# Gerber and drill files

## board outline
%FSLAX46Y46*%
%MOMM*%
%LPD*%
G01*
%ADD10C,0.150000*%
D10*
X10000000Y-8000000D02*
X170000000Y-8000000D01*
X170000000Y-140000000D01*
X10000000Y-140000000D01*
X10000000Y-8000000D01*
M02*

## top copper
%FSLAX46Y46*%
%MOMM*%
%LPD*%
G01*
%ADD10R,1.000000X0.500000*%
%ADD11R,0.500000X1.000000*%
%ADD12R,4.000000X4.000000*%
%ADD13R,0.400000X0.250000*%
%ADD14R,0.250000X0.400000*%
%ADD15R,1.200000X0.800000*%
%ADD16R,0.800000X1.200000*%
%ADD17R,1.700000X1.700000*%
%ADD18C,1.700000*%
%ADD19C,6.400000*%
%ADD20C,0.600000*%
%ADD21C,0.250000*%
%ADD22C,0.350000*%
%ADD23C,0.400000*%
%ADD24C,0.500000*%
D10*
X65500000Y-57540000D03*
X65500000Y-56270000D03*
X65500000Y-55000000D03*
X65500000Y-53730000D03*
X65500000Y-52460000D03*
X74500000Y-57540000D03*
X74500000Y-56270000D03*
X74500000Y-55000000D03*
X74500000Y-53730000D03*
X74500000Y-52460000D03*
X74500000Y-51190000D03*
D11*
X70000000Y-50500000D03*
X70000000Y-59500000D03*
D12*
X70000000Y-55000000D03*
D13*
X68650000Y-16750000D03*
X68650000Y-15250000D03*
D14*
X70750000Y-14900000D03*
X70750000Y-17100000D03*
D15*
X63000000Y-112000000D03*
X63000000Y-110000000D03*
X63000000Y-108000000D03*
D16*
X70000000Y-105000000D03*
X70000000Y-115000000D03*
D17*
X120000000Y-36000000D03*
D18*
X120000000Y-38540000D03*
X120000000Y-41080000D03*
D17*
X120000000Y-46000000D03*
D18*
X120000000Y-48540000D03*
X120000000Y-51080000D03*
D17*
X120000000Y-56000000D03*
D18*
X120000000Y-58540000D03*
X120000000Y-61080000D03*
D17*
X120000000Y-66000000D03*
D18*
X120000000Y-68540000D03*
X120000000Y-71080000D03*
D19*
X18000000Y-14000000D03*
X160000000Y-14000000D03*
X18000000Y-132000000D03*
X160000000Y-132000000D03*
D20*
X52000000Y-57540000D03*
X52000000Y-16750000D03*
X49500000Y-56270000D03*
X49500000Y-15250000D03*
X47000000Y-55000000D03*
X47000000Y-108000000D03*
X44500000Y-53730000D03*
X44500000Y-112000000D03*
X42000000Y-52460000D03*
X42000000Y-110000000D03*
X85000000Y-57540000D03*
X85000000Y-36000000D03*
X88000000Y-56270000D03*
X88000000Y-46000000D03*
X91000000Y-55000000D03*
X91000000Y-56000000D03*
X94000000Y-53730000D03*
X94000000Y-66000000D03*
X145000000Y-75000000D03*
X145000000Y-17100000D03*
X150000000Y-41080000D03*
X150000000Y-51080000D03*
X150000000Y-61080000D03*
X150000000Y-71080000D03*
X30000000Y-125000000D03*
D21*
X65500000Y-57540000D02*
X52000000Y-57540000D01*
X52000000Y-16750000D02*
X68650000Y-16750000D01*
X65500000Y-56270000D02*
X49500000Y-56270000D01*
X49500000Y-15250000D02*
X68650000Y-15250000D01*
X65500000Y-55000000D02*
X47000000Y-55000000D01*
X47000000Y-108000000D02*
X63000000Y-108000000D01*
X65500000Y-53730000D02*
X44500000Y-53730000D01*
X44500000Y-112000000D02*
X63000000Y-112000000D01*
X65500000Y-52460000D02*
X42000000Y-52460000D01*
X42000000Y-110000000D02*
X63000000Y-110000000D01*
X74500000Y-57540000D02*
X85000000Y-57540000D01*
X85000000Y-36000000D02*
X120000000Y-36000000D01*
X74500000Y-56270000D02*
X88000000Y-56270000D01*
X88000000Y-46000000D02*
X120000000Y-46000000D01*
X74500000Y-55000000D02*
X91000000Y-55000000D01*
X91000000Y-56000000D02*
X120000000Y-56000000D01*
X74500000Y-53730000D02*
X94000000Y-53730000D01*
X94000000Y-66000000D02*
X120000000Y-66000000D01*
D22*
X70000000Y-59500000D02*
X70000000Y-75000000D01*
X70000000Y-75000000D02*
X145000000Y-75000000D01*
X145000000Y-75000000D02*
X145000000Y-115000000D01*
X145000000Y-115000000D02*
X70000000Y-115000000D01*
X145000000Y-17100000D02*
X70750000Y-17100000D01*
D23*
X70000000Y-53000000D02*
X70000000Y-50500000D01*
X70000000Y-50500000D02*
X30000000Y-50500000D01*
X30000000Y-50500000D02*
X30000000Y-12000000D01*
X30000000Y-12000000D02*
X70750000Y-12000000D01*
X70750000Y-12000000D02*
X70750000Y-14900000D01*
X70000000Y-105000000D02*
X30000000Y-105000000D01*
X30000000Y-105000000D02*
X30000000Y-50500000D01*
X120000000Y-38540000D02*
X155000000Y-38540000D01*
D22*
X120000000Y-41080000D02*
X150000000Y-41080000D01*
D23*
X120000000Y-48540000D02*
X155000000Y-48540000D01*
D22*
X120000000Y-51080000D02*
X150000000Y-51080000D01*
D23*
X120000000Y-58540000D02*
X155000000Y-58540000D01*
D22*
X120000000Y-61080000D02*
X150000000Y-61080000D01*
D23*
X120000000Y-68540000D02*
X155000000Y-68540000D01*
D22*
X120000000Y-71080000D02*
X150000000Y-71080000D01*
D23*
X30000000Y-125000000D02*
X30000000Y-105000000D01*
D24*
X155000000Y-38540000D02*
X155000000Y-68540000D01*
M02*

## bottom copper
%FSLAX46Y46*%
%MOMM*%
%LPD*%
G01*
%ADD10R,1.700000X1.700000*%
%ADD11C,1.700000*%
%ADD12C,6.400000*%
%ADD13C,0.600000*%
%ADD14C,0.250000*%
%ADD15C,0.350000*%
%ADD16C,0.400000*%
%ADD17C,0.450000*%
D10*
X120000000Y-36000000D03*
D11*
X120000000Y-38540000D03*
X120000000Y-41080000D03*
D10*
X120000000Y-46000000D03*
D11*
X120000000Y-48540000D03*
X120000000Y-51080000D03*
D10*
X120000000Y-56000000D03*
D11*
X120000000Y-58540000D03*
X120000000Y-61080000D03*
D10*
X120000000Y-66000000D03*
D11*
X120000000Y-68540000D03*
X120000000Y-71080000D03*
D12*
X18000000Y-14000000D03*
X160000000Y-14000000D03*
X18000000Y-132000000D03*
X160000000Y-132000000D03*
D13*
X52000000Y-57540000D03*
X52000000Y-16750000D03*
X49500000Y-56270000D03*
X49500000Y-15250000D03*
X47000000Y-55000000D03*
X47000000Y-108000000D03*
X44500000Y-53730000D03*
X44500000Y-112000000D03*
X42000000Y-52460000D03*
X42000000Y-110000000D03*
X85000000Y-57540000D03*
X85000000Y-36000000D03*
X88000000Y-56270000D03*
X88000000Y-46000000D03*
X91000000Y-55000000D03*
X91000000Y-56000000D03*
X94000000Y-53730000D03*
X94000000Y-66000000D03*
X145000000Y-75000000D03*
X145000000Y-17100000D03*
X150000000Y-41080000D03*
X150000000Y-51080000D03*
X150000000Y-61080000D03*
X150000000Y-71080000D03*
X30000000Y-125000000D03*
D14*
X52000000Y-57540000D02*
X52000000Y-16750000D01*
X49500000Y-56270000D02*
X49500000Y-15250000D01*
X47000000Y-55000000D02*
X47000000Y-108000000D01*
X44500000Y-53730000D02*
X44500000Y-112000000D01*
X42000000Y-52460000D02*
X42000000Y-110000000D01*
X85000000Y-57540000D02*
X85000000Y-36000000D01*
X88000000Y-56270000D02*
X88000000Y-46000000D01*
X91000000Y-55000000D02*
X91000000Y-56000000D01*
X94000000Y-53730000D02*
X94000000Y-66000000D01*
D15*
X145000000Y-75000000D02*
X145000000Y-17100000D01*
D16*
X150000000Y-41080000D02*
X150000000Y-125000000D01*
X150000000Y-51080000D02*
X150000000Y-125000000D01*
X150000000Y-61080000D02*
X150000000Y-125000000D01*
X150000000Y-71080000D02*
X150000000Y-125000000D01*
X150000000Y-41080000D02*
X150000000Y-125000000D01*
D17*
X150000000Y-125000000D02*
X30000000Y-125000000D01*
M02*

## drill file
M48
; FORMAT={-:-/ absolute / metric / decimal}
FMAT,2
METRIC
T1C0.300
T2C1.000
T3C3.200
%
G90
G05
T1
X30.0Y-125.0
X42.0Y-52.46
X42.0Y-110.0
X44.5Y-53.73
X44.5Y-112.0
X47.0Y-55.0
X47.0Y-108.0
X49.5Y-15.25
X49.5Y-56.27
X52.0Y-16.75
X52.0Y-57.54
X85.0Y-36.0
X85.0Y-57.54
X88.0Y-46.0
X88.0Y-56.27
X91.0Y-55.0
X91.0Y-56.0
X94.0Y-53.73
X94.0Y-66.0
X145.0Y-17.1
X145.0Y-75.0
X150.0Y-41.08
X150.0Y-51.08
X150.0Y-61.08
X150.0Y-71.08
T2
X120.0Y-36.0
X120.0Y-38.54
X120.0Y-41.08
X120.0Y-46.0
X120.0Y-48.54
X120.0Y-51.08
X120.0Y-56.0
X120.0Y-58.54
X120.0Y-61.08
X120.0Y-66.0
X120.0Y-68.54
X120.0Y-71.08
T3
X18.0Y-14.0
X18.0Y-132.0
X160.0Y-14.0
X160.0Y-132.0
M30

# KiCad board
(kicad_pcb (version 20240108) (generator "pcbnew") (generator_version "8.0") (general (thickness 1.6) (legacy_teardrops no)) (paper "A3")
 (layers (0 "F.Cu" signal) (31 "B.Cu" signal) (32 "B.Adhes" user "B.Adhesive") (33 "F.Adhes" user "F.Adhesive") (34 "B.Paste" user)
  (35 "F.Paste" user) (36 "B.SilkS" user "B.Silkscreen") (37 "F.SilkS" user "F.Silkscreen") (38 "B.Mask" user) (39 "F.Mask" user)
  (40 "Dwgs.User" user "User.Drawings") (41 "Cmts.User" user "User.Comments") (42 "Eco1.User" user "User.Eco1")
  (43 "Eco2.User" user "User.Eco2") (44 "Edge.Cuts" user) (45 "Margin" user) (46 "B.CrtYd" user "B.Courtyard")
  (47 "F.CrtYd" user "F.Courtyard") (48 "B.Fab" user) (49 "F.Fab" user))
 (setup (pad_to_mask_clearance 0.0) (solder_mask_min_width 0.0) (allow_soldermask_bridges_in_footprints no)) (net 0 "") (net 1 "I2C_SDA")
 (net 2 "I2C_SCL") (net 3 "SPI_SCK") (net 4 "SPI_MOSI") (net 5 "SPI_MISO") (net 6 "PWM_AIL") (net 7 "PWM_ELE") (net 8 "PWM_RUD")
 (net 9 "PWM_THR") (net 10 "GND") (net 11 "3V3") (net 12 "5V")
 (gr_rect (start 10 8) (end 170 140) (stroke (width 0.15) (type solid)) (fill none) (layer "Edge.Cuts"))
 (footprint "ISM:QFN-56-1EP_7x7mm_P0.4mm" (layer "F.Cu") (at 70 55)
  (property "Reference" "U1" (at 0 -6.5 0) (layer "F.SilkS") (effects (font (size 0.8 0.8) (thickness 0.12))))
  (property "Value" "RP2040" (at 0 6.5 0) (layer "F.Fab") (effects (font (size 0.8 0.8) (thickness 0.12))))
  (pad "1" smd rect (at -4.5 2.54) (size 1.0 0.5) (layers "F.Cu" "F.Paste" "F.Mask") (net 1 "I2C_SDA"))
  (pad "2" smd rect (at -4.5 1.27) (size 1.0 0.5) (layers "F.Cu" "F.Paste" "F.Mask") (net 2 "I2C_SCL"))
  (pad "3" smd rect (at -4.5 0) (size 1.0 0.5) (layers "F.Cu" "F.Paste" "F.Mask") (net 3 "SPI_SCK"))
  (pad "4" smd rect (at -4.5 -1.27) (size 1.0 0.5) (layers "F.Cu" "F.Paste" "F.Mask") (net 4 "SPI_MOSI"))
  (pad "5" smd rect (at -4.5 -2.54) (size 1.0 0.5) (layers "F.Cu" "F.Paste" "F.Mask") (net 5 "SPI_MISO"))
  (pad "6" smd rect (at 4.5 2.54) (size 1.0 0.5) (layers "F.Cu" "F.Paste" "F.Mask") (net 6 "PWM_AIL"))
  (pad "7" smd rect (at 4.5 1.27) (size 1.0 0.5) (layers "F.Cu" "F.Paste" "F.Mask") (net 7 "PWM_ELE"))
  (pad "8" smd rect (at 4.5 0) (size 1.0 0.5) (layers "F.Cu" "F.Paste" "F.Mask") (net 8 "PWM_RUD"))
  (pad "9" smd rect (at 4.5 -1.27) (size 1.0 0.5) (layers "F.Cu" "F.Paste" "F.Mask") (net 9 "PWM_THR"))
  (pad "12" smd rect (at 4.5 -2.54) (size 1.0 0.5) (layers "F.Cu" "F.Paste" "F.Mask"))
  (pad "13" smd rect (at 4.5 -3.81) (size 1.0 0.5) (layers "F.Cu" "F.Paste" "F.Mask"))
  (pad "10" smd rect (at 0 -4.5) (size 0.5 1.0) (layers "F.Cu" "F.Paste" "F.Mask") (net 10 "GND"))
  (pad "11" smd rect (at 0 4.5) (size 0.5 1.0) (layers "F.Cu" "F.Paste" "F.Mask") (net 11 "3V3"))
  (pad "EP" smd rect (at 0 0) (size 4 4) (layers "F.Cu" "F.Paste" "F.Mask") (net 10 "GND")))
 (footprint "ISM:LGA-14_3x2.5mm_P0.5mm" (layer "F.Cu") (at 70 16)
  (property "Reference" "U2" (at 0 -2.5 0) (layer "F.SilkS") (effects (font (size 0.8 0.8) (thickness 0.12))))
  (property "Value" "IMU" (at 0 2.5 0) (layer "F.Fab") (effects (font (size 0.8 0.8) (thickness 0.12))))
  (pad "1" smd rect (at -1.35 0.75) (size 0.4 0.25) (layers "F.Cu" "F.Paste" "F.Mask") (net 1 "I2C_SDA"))
  (pad "2" smd rect (at -1.35 -0.75) (size 0.4 0.25) (layers "F.Cu" "F.Paste" "F.Mask") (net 2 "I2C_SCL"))
  (pad "3" smd rect (at 0.75 -1.1) (size 0.25 0.4) (layers "F.Cu" "F.Paste" "F.Mask") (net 10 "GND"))
  (pad "4" smd rect (at 0.75 1.1) (size 0.25 0.4) (layers "F.Cu" "F.Paste" "F.Mask") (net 11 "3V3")))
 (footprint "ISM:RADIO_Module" (layer "F.Cu") (at 70 110)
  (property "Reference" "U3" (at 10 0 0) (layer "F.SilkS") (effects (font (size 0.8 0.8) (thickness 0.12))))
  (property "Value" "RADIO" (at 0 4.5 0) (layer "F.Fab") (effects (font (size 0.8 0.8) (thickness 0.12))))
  (pad "1" smd rect (at -7 2) (size 1.2 0.8) (layers "F.Cu" "F.Paste" "F.Mask") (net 4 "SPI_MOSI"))
  (pad "2" smd rect (at -7 0) (size 1.2 0.8) (layers "F.Cu" "F.Paste" "F.Mask") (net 5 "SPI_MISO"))
  (pad "3" smd rect (at -7 -2) (size 1.2 0.8) (layers "F.Cu" "F.Paste" "F.Mask") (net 3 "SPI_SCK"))
  (pad "4" smd rect (at 0 -5) (size 0.8 1.2) (layers "F.Cu" "F.Paste" "F.Mask") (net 10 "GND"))
  (pad "5" smd rect (at 0 5) (size 0.8 1.2) (layers "F.Cu" "F.Paste" "F.Mask") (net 11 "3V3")))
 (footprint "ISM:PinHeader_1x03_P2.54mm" (layer "F.Cu") (at 120 36)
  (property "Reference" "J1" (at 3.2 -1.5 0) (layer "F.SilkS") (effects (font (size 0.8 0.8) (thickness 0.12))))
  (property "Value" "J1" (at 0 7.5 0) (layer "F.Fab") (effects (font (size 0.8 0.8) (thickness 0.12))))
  (pad "1" thru_hole rect (at 0 0) (size 1.7 1.7) (drill 1.0) (layers "*.Cu" "*.Mask") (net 6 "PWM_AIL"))
  (pad "2" thru_hole circle (at 0 2.54) (size 1.7 1.7) (drill 1.0) (layers "*.Cu" "*.Mask") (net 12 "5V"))
  (pad "3" thru_hole circle (at 0 5.08) (size 1.7 1.7) (drill 1.0) (layers "*.Cu" "*.Mask") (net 10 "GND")))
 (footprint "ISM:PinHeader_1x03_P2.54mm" (layer "F.Cu") (at 120 46)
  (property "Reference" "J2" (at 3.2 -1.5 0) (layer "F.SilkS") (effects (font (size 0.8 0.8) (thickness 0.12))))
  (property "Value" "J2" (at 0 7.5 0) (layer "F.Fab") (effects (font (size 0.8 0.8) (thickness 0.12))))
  (pad "1" thru_hole rect (at 0 0) (size 1.7 1.7) (drill 1.0) (layers "*.Cu" "*.Mask") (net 7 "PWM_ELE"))
  (pad "2" thru_hole circle (at 0 2.54) (size 1.7 1.7) (drill 1.0) (layers "*.Cu" "*.Mask") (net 12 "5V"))
  (pad "3" thru_hole circle (at 0 5.08) (size 1.7 1.7) (drill 1.0) (layers "*.Cu" "*.Mask") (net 10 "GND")))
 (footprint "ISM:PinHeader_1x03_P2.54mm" (layer "F.Cu") (at 120 56)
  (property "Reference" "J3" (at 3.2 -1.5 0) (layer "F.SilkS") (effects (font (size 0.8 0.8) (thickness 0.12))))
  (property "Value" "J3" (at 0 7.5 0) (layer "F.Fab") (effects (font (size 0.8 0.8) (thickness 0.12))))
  (pad "1" thru_hole rect (at 0 0) (size 1.7 1.7) (drill 1.0) (layers "*.Cu" "*.Mask") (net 8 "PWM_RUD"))
  (pad "2" thru_hole circle (at 0 2.54) (size 1.7 1.7) (drill 1.0) (layers "*.Cu" "*.Mask") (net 12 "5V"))
  (pad "3" thru_hole circle (at 0 5.08) (size 1.7 1.7) (drill 1.0) (layers "*.Cu" "*.Mask") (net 10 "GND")))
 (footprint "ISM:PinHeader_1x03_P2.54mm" (layer "F.Cu") (at 120 66)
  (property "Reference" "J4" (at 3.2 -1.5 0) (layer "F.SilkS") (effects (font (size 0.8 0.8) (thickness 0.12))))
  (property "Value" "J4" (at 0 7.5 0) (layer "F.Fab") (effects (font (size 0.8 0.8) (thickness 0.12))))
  (pad "1" thru_hole rect (at 0 0) (size 1.7 1.7) (drill 1.0) (layers "*.Cu" "*.Mask") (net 9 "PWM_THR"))
  (pad "2" thru_hole circle (at 0 2.54) (size 1.7 1.7) (drill 1.0) (layers "*.Cu" "*.Mask") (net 12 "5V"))
  (pad "3" thru_hole circle (at 0 5.08) (size 1.7 1.7) (drill 1.0) (layers "*.Cu" "*.Mask") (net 10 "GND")))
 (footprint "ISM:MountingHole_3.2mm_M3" (layer "F.Cu") (at 18 14)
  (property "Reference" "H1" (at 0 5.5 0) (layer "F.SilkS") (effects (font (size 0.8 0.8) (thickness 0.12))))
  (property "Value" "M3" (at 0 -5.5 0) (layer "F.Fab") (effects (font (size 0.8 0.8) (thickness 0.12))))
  (pad "" thru_hole circle (at 0 0) (size 6.4 6.4) (drill 3.2) (layers "*.Cu" "*.Mask")))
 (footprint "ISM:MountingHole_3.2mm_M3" (layer "F.Cu") (at 160 14)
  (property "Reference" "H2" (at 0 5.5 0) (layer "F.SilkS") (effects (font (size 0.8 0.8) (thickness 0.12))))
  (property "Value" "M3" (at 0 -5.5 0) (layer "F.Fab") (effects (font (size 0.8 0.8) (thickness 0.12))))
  (pad "" thru_hole circle (at 0 0) (size 6.4 6.4) (drill 3.2) (layers "*.Cu" "*.Mask")))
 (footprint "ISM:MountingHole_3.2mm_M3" (layer "F.Cu") (at 18 132)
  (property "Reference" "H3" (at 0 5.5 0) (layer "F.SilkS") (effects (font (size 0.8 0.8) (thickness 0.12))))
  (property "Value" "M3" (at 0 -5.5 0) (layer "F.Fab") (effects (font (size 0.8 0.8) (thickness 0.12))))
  (pad "" thru_hole circle (at 0 0) (size 6.4 6.4) (drill 3.2) (layers "*.Cu" "*.Mask")))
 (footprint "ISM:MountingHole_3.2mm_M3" (layer "F.Cu") (at 160 132)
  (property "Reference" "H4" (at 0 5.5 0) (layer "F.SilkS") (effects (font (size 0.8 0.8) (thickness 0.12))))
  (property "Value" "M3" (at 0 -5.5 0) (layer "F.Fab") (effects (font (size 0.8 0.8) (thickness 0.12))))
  (pad "" thru_hole circle (at 0 0) (size 6.4 6.4) (drill 3.2) (layers "*.Cu" "*.Mask")))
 (segment (start 65.5 57.54) (end 52.0 57.54) (width 0.25) (layer "F.Cu") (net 1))
 (segment (start 52.0 57.54) (end 52.0 16.75) (width 0.25) (layer "B.Cu") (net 1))
 (segment (start 52.0 16.75) (end 68.65 16.75) (width 0.25) (layer "F.Cu") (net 1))
 (segment (start 65.5 56.27) (end 49.5 56.27) (width 0.25) (layer "F.Cu") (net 2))
 (segment (start 49.5 56.27) (end 49.5 15.25) (width 0.25) (layer "B.Cu") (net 2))
 (segment (start 49.5 15.25) (end 68.65 15.25) (width 0.25) (layer "F.Cu") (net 2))
 (segment (start 65.5 55) (end 47.0 55) (width 0.25) (layer "F.Cu") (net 3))
 (segment (start 47.0 55) (end 47.0 108) (width 0.25) (layer "B.Cu") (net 3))
 (segment (start 47.0 108) (end 63 108) (width 0.25) (layer "F.Cu") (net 3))
 (segment (start 65.5 53.73) (end 44.5 53.73) (width 0.25) (layer "F.Cu") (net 4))
 (segment (start 44.5 53.73) (end 44.5 112) (width 0.25) (layer "B.Cu") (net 4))
 (segment (start 44.5 112) (end 63 112) (width 0.25) (layer "F.Cu") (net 4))
 (segment (start 65.5 52.46) (end 42.0 52.46) (width 0.25) (layer "F.Cu") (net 5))
 (segment (start 42.0 52.46) (end 42.0 110) (width 0.25) (layer "B.Cu") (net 5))
 (segment (start 42.0 110) (end 63 110) (width 0.25) (layer "F.Cu") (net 5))
 (segment (start 74.5 57.54) (end 85 57.54) (width 0.25) (layer "F.Cu") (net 6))
 (segment (start 85 57.54) (end 85 36) (width 0.25) (layer "B.Cu") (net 6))
 (segment (start 85 36) (end 120 36) (width 0.25) (layer "F.Cu") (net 6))
 (segment (start 74.5 56.27) (end 88 56.27) (width 0.25) (layer "F.Cu") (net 7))
 (segment (start 88 56.27) (end 88 46) (width 0.25) (layer "B.Cu") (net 7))
 (segment (start 88 46) (end 120 46) (width 0.25) (layer "F.Cu") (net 7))
 (segment (start 74.5 55) (end 91 55) (width 0.25) (layer "F.Cu") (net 8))
 (segment (start 91 55) (end 91 56) (width 0.25) (layer "B.Cu") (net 8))
 (segment (start 91 56) (end 120 56) (width 0.25) (layer "F.Cu") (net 8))
 (segment (start 74.5 53.73) (end 94 53.73) (width 0.25) (layer "F.Cu") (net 9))
 (segment (start 94 53.73) (end 94 66) (width 0.25) (layer "B.Cu") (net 9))
 (segment (start 94 66) (end 120 66) (width 0.25) (layer "F.Cu") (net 9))
 (segment (start 70 59.5) (end 70 75) (width 0.35) (layer "F.Cu") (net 11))
 (segment (start 70 75) (end 145 75) (width 0.35) (layer "F.Cu") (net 11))
 (segment (start 145 75) (end 145 115) (width 0.35) (layer "F.Cu") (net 11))
 (segment (start 145 115) (end 70 115) (width 0.35) (layer "F.Cu") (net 11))
 (segment (start 145 75) (end 145 17.1) (width 0.35) (layer "B.Cu") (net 11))
 (segment (start 145 17.1) (end 70.75 17.1) (width 0.35) (layer "F.Cu") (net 11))
 (segment (start 70 53) (end 70 50.5) (width 0.4) (layer "F.Cu") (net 10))
 (segment (start 70 50.5) (end 30 50.5) (width 0.4) (layer "F.Cu") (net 10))
 (segment (start 30 50.5) (end 30 12) (width 0.4) (layer "F.Cu") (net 10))
 (segment (start 30 12) (end 70.75 12) (width 0.4) (layer "F.Cu") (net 10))
 (segment (start 70.75 12) (end 70.75 14.9) (width 0.4) (layer "F.Cu") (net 10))
 (segment (start 70 105) (end 30 105) (width 0.4) (layer "F.Cu") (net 10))
 (segment (start 30 105) (end 30 50.5) (width 0.4) (layer "F.Cu") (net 10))
 (segment (start 120 38.54) (end 155 38.54) (width 0.4) (layer "F.Cu") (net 12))
 (segment (start 120 41.08) (end 150 41.08) (width 0.35) (layer "F.Cu") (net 10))
 (segment (start 150 41.08) (end 150 125) (width 0.4) (layer "B.Cu") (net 10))
 (segment (start 120 48.54) (end 155 48.54) (width 0.4) (layer "F.Cu") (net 12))
 (segment (start 120 51.08) (end 150 51.08) (width 0.35) (layer "F.Cu") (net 10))
 (segment (start 150 51.08) (end 150 125) (width 0.4) (layer "B.Cu") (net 10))
 (segment (start 120 58.54) (end 155 58.54) (width 0.4) (layer "F.Cu") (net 12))
 (segment (start 120 61.08) (end 150 61.08) (width 0.35) (layer "F.Cu") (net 10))
 (segment (start 150 61.08) (end 150 125) (width 0.4) (layer "B.Cu") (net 10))
 (segment (start 120 68.54) (end 155 68.54) (width 0.4) (layer "F.Cu") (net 12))
 (segment (start 120 71.08) (end 150 71.08) (width 0.35) (layer "F.Cu") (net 10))
 (segment (start 150 71.08) (end 150 125) (width 0.4) (layer "B.Cu") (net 10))
 (segment (start 150 41.08) (end 150 125) (width 0.4) (layer "B.Cu") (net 10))
 (segment (start 150 125) (end 30 125) (width 0.45) (layer "B.Cu") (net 10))
 (segment (start 30 125) (end 30 105) (width 0.4) (layer "F.Cu") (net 10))
 (segment (start 155 38.54) (end 155 68.54) (width 0.5) (layer "F.Cu") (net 12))
 (via (at 52.0 57.54) (size 0.6) (drill 0.3) (layers "F.Cu" "B.Cu") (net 1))
 (via (at 52.0 16.75) (size 0.6) (drill 0.3) (layers "F.Cu" "B.Cu") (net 1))
 (via (at 49.5 56.27) (size 0.6) (drill 0.3) (layers "F.Cu" "B.Cu") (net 2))
 (via (at 49.5 15.25) (size 0.6) (drill 0.3) (layers "F.Cu" "B.Cu") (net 2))
 (via (at 47.0 55) (size 0.6) (drill 0.3) (layers "F.Cu" "B.Cu") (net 3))
 (via (at 47.0 108) (size 0.6) (drill 0.3) (layers "F.Cu" "B.Cu") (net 3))
 (via (at 44.5 53.73) (size 0.6) (drill 0.3) (layers "F.Cu" "B.Cu") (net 4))
 (via (at 44.5 112) (size 0.6) (drill 0.3) (layers "F.Cu" "B.Cu") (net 4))
 (via (at 42.0 52.46) (size 0.6) (drill 0.3) (layers "F.Cu" "B.Cu") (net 5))
 (via (at 42.0 110) (size 0.6) (drill 0.3) (layers "F.Cu" "B.Cu") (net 5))
 (via (at 85 57.54) (size 0.6) (drill 0.3) (layers "F.Cu" "B.Cu") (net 6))
 (via (at 85 36) (size 0.6) (drill 0.3) (layers "F.Cu" "B.Cu") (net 6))
 (via (at 88 56.27) (size 0.6) (drill 0.3) (layers "F.Cu" "B.Cu") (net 7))
 (via (at 88 46) (size 0.6) (drill 0.3) (layers "F.Cu" "B.Cu") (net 7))
 (via (at 91 55) (size 0.6) (drill 0.3) (layers "F.Cu" "B.Cu") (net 8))
 (via (at 91 56) (size 0.6) (drill 0.3) (layers "F.Cu" "B.Cu") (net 8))
 (via (at 94 53.73) (size 0.6) (drill 0.3) (layers "F.Cu" "B.Cu") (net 9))
 (via (at 94 66) (size 0.6) (drill 0.3) (layers "F.Cu" "B.Cu") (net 9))
 (via (at 145 75) (size 0.6) (drill 0.3) (layers "F.Cu" "B.Cu") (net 11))
 (via (at 145 17.1) (size 0.6) (drill 0.3) (layers "F.Cu" "B.Cu") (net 11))
 (via (at 150 41.08) (size 0.6) (drill 0.3) (layers "F.Cu" "B.Cu") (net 10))
 (via (at 150 51.08) (size 0.6) (drill 0.3) (layers "F.Cu" "B.Cu") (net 10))
 (via (at 150 61.08) (size 0.6) (drill 0.3) (layers "F.Cu" "B.Cu") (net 10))
 (via (at 150 71.08) (size 0.6) (drill 0.3) (layers "F.Cu" "B.Cu") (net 10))
 (via (at 30 125) (size 0.6) (drill 0.3) (layers "F.Cu" "B.Cu") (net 10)))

